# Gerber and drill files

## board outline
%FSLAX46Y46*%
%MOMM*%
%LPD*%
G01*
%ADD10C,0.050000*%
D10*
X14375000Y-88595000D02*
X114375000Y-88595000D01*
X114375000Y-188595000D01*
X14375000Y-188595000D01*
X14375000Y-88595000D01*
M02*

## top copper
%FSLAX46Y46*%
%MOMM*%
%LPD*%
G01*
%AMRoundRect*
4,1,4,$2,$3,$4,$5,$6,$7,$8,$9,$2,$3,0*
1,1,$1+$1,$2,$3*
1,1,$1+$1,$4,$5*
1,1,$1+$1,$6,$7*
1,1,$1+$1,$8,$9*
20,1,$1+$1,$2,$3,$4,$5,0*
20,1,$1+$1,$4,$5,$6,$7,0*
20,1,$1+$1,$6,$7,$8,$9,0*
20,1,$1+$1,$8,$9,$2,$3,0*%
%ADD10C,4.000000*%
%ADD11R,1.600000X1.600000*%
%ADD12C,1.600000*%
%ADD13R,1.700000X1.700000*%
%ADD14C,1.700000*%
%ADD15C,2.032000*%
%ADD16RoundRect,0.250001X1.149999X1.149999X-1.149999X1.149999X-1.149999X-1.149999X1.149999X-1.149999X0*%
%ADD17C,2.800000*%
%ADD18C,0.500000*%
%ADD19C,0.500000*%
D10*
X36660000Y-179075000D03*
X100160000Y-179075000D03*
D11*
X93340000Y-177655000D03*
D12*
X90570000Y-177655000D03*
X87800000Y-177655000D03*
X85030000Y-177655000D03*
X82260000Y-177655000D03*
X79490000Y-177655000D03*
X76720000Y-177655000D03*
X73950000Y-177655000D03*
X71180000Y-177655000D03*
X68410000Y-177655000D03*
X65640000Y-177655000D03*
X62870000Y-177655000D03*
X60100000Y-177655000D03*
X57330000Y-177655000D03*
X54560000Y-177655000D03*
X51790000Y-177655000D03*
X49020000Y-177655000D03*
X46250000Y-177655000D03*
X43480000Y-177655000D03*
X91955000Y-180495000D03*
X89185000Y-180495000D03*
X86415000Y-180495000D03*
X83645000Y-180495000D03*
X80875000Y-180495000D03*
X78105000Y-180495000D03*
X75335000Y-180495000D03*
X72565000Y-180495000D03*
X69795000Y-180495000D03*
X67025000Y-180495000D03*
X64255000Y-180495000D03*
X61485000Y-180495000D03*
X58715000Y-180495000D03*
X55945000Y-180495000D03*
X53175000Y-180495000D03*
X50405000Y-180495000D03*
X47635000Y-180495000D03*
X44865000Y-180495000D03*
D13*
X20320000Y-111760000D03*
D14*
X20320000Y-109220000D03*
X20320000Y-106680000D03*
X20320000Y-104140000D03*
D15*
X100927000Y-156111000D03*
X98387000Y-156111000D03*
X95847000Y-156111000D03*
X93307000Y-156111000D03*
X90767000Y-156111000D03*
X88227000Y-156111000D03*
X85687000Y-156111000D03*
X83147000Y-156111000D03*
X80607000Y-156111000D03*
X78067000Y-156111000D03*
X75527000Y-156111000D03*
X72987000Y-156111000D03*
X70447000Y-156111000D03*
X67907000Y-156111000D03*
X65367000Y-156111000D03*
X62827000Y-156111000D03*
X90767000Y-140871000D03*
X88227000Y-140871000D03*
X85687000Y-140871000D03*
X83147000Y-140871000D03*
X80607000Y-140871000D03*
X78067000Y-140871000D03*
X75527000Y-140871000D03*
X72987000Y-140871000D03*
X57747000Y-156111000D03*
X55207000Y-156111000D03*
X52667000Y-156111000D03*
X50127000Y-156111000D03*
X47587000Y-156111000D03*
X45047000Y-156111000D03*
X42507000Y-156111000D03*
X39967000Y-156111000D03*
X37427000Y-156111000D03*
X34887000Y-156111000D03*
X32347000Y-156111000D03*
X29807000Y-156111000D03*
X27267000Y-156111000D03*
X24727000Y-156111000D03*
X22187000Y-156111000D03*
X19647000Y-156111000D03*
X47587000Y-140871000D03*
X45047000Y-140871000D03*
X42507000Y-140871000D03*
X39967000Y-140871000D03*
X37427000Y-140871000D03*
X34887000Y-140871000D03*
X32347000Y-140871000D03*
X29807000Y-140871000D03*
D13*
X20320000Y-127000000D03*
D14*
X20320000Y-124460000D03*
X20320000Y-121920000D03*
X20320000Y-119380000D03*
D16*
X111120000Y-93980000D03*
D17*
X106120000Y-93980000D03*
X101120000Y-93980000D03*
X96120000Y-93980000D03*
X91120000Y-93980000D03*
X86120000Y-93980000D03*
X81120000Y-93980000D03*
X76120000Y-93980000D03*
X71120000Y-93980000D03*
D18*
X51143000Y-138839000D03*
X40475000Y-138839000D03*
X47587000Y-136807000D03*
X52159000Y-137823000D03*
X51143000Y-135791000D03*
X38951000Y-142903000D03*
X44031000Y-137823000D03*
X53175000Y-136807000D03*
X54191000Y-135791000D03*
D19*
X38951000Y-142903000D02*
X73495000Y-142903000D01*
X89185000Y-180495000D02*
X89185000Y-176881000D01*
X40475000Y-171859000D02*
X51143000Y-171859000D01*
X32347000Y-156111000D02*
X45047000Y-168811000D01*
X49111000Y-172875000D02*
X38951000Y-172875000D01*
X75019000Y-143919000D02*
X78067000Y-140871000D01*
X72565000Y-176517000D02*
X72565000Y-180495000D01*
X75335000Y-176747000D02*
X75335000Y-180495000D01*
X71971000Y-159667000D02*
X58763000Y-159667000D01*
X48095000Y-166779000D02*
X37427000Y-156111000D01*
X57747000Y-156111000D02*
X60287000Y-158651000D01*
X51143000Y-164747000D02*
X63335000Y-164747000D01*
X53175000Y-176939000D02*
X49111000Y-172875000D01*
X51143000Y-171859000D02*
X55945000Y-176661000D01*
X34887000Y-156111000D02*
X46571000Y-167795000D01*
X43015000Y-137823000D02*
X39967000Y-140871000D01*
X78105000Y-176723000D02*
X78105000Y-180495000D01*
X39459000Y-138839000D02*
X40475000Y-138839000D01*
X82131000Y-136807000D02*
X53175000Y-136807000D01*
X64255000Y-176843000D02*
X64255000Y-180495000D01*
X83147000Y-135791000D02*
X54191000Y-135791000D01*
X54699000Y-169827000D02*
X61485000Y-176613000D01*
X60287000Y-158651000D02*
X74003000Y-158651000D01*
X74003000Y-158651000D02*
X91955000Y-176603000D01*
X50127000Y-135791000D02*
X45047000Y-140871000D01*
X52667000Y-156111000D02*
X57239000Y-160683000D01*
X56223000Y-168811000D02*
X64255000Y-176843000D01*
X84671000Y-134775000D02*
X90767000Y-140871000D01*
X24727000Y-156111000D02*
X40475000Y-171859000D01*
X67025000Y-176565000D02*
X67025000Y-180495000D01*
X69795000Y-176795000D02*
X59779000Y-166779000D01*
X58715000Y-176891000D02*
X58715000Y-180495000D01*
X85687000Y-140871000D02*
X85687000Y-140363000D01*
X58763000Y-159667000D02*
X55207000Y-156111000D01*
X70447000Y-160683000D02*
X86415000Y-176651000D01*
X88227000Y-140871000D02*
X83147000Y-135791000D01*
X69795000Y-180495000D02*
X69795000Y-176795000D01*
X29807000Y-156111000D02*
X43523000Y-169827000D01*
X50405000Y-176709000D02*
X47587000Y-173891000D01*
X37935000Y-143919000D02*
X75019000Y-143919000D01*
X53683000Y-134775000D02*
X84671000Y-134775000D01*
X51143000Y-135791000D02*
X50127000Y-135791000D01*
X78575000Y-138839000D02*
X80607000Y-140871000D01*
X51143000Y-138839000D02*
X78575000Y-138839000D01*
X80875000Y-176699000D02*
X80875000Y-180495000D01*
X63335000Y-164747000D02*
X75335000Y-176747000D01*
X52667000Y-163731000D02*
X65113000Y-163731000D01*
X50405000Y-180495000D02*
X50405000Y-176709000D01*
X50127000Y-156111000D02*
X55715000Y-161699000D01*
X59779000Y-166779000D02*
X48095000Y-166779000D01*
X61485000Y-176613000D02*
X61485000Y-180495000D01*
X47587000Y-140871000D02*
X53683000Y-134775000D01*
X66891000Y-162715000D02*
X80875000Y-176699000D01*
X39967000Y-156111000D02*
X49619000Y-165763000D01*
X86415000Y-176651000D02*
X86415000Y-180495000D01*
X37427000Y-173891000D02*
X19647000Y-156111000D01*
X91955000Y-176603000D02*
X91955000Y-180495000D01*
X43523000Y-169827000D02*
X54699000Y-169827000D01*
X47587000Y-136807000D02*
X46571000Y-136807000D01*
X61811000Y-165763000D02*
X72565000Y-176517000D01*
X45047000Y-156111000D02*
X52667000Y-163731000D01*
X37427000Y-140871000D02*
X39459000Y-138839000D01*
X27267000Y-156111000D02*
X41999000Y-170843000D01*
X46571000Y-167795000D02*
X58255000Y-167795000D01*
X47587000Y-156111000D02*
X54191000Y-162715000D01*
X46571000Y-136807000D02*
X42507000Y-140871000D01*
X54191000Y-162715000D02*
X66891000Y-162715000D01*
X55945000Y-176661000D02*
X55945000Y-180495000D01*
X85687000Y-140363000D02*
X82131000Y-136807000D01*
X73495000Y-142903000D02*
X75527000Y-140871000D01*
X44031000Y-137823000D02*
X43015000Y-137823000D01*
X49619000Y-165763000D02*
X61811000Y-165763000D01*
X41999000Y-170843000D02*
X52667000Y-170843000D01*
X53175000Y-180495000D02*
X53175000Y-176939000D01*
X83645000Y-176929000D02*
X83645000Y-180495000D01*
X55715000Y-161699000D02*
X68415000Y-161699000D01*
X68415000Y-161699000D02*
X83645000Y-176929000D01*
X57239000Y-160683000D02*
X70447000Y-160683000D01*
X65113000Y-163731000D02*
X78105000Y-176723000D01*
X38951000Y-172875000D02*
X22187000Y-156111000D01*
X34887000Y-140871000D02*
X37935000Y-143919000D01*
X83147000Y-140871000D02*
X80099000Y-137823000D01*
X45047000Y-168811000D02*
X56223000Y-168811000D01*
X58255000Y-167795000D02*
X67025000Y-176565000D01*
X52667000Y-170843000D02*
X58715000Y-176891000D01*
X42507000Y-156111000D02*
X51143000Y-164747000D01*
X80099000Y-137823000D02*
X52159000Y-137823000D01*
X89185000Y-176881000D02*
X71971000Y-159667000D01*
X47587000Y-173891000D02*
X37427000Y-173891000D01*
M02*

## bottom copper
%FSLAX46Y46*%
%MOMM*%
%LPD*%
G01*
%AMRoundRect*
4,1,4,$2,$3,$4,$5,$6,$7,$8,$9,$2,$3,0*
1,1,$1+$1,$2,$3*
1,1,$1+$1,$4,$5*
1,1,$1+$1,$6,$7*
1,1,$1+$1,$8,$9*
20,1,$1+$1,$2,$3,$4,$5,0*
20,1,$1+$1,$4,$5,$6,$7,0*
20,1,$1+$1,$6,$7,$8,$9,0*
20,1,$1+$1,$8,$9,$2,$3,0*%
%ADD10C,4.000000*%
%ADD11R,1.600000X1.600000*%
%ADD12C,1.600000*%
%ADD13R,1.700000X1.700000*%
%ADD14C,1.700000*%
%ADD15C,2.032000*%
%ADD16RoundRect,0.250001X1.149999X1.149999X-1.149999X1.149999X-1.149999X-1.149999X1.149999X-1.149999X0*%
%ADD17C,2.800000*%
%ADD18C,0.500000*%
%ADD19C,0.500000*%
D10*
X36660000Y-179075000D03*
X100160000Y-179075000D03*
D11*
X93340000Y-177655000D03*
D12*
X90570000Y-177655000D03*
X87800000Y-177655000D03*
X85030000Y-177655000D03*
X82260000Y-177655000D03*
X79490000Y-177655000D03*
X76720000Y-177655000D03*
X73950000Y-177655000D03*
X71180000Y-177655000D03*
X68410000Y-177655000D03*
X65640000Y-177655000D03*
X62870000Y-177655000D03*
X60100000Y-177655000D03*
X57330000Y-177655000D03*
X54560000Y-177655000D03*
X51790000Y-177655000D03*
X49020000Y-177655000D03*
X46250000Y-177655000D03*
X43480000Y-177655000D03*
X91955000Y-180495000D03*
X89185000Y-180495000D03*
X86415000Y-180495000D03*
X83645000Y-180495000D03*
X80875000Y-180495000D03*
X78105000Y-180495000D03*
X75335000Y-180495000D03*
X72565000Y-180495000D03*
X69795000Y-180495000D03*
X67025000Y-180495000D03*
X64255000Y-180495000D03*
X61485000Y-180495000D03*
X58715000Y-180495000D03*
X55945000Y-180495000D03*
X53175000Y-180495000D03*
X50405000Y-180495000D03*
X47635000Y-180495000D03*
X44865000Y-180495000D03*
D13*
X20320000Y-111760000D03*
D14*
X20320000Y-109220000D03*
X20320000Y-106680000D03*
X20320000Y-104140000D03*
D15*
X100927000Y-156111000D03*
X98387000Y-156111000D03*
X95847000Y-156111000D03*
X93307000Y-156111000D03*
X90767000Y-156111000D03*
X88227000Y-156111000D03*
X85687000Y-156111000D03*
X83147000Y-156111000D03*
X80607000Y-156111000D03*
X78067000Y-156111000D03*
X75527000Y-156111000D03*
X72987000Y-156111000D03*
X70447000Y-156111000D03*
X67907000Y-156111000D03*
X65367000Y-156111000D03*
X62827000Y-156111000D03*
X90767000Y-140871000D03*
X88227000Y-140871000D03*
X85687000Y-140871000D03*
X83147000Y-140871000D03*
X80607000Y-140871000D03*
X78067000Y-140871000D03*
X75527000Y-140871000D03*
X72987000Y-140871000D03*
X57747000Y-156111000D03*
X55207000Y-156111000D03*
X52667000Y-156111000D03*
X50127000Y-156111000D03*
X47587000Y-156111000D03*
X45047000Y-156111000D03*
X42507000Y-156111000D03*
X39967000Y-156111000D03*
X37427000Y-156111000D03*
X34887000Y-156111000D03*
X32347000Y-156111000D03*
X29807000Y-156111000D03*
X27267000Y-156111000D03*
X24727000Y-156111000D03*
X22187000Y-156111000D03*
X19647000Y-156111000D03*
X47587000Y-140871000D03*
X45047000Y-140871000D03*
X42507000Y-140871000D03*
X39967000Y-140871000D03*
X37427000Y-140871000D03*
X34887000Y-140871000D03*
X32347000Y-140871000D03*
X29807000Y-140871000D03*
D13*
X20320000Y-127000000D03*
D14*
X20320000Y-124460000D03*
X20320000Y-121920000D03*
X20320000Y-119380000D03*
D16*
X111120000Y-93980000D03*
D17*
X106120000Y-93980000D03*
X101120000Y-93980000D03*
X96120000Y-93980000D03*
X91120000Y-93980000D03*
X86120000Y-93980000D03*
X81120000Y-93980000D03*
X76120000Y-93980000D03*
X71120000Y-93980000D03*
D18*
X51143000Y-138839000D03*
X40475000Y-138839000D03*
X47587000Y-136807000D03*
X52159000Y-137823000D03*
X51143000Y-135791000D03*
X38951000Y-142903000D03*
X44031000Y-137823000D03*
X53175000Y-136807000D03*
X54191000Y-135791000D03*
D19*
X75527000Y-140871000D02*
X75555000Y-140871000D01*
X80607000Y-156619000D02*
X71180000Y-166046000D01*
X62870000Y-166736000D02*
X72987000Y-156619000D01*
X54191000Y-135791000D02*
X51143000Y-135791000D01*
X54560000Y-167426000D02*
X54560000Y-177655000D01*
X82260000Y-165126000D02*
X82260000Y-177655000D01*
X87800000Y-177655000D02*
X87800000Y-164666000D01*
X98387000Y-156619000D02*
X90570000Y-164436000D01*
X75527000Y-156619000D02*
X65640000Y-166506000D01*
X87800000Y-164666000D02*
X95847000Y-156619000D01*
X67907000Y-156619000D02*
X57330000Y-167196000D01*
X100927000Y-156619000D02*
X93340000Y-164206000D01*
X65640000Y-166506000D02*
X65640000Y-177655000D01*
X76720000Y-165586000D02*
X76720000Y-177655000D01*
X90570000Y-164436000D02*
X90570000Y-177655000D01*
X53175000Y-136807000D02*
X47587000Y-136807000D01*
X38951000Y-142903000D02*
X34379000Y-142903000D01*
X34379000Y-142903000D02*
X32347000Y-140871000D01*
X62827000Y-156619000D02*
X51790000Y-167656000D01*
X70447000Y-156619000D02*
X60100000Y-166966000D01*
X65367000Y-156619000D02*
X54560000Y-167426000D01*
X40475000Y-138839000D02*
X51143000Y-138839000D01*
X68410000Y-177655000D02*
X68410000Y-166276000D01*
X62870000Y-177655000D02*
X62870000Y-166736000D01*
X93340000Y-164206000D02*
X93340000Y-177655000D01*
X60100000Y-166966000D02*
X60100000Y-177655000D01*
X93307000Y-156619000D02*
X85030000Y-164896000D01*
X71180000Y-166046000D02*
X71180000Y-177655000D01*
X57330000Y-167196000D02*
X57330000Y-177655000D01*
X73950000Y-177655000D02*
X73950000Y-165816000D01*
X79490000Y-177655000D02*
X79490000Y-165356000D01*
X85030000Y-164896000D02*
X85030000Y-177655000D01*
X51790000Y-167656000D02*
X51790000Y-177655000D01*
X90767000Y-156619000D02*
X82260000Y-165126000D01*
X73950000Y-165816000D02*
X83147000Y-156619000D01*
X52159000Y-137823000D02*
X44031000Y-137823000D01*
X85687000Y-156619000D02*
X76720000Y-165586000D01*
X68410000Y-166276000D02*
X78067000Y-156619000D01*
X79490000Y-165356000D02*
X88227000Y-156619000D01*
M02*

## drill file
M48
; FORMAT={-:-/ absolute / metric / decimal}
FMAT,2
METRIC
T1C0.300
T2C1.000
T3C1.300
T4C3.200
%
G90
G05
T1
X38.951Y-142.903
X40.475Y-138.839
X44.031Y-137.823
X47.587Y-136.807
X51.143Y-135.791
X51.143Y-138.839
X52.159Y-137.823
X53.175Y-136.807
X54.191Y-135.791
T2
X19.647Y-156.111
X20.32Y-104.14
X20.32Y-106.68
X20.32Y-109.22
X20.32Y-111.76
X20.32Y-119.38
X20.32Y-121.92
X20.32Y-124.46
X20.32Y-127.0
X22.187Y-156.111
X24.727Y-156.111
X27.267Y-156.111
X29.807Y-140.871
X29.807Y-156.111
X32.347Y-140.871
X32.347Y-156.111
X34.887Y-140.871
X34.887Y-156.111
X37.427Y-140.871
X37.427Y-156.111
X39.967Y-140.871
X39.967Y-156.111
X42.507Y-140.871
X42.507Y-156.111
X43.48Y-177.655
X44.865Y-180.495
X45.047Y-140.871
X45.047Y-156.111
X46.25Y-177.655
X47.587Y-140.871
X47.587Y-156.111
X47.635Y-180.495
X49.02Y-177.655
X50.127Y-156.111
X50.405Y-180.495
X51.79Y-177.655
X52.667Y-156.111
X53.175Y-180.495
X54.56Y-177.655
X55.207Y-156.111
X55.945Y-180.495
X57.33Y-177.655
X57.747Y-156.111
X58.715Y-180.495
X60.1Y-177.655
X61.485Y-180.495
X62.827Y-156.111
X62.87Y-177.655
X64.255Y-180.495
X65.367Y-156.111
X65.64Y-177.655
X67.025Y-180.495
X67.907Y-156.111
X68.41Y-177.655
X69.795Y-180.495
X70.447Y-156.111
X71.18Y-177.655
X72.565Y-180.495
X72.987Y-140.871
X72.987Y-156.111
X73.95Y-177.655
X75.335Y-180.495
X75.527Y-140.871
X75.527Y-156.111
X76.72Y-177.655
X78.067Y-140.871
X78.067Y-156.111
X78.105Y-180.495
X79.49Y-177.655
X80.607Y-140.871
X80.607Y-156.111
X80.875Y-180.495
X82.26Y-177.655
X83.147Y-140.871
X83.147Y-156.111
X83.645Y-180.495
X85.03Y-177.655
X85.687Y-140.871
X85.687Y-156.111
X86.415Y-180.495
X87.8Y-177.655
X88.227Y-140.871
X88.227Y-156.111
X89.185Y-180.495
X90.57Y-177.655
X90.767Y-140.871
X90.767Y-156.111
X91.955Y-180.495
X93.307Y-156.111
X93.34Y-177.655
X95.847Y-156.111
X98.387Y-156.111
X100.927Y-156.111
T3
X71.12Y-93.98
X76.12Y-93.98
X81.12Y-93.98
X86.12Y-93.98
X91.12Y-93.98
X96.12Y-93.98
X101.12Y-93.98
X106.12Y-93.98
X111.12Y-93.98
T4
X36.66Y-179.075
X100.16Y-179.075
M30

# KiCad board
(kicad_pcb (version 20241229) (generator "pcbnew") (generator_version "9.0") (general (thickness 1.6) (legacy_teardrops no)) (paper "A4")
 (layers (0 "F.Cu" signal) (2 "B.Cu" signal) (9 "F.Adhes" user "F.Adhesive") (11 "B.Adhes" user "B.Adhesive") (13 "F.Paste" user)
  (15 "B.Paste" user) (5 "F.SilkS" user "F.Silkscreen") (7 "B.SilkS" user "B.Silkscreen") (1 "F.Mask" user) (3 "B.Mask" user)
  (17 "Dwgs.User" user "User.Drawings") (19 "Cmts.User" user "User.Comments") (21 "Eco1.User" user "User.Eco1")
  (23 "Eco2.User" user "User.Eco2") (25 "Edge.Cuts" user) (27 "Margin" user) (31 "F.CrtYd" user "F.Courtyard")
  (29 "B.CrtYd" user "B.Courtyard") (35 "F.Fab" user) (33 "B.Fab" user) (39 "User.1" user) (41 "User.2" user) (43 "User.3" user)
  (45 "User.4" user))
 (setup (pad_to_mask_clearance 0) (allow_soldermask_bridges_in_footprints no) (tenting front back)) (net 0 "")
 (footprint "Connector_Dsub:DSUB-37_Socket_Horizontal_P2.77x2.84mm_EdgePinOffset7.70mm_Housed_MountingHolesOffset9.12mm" (layer "F.Cu")
  (at 93.34 177.655)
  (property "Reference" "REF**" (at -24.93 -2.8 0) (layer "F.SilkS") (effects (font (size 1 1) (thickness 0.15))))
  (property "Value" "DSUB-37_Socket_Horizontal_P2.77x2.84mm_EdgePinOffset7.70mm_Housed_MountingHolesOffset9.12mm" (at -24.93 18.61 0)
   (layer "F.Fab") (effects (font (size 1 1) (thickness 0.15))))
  (pad "0" thru_hole circle (at -56.68 1.42) (size 4 4) (drill 3.2) (layers "*.Cu" "*.Mask") (remove_unused_layers no))
  (pad "0" thru_hole circle (at 6.82 1.42) (size 4 4) (drill 3.2) (layers "*.Cu" "*.Mask") (remove_unused_layers no))
  (pad "1" thru_hole rect (at 0 0) (size 1.6 1.6) (drill 1) (layers "*.Cu" "*.Mask") (remove_unused_layers no))
  (pad "2" thru_hole circle (at -2.77 0) (size 1.6 1.6) (drill 1) (layers "*.Cu" "*.Mask") (remove_unused_layers no))
  (pad "3" thru_hole circle (at -5.54 0) (size 1.6 1.6) (drill 1) (layers "*.Cu" "*.Mask") (remove_unused_layers no))
  (pad "4" thru_hole circle (at -8.31 0) (size 1.6 1.6) (drill 1) (layers "*.Cu" "*.Mask") (remove_unused_layers no))
  (pad "5" thru_hole circle (at -11.08 0) (size 1.6 1.6) (drill 1) (layers "*.Cu" "*.Mask") (remove_unused_layers no))
  (pad "6" thru_hole circle (at -13.85 0) (size 1.6 1.6) (drill 1) (layers "*.Cu" "*.Mask") (remove_unused_layers no))
  (pad "7" thru_hole circle (at -16.62 0) (size 1.6 1.6) (drill 1) (layers "*.Cu" "*.Mask") (remove_unused_layers no))
  (pad "8" thru_hole circle (at -19.39 0) (size 1.6 1.6) (drill 1) (layers "*.Cu" "*.Mask") (remove_unused_layers no))
  (pad "9" thru_hole circle (at -22.16 0) (size 1.6 1.6) (drill 1) (layers "*.Cu" "*.Mask") (remove_unused_layers no))
  (pad "10" thru_hole circle (at -24.93 0) (size 1.6 1.6) (drill 1) (layers "*.Cu" "*.Mask") (remove_unused_layers no))
  (pad "11" thru_hole circle (at -27.7 0) (size 1.6 1.6) (drill 1) (layers "*.Cu" "*.Mask") (remove_unused_layers no))
  (pad "12" thru_hole circle (at -30.47 0) (size 1.6 1.6) (drill 1) (layers "*.Cu" "*.Mask") (remove_unused_layers no))
  (pad "13" thru_hole circle (at -33.24 0) (size 1.6 1.6) (drill 1) (layers "*.Cu" "*.Mask") (remove_unused_layers no))
  (pad "14" thru_hole circle (at -36.01 0) (size 1.6 1.6) (drill 1) (layers "*.Cu" "*.Mask") (remove_unused_layers no))
  (pad "15" thru_hole circle (at -38.78 0) (size 1.6 1.6) (drill 1) (layers "*.Cu" "*.Mask") (remove_unused_layers no))
  (pad "16" thru_hole circle (at -41.55 0) (size 1.6 1.6) (drill 1) (layers "*.Cu" "*.Mask") (remove_unused_layers no))
  (pad "17" thru_hole circle (at -44.32 0) (size 1.6 1.6) (drill 1) (layers "*.Cu" "*.Mask") (remove_unused_layers no))
  (pad "18" thru_hole circle (at -47.09 0) (size 1.6 1.6) (drill 1) (layers "*.Cu" "*.Mask") (remove_unused_layers no))
  (pad "19" thru_hole circle (at -49.86 0) (size 1.6 1.6) (drill 1) (layers "*.Cu" "*.Mask") (remove_unused_layers no))
  (pad "20" thru_hole circle (at -1.385 2.84) (size 1.6 1.6) (drill 1) (layers "*.Cu" "*.Mask") (remove_unused_layers no))
  (pad "21" thru_hole circle (at -4.155 2.84) (size 1.6 1.6) (drill 1) (layers "*.Cu" "*.Mask") (remove_unused_layers no))
  (pad "22" thru_hole circle (at -6.925 2.84) (size 1.6 1.6) (drill 1) (layers "*.Cu" "*.Mask") (remove_unused_layers no))
  (pad "23" thru_hole circle (at -9.695 2.84) (size 1.6 1.6) (drill 1) (layers "*.Cu" "*.Mask") (remove_unused_layers no))
  (pad "24" thru_hole circle (at -12.465 2.84) (size 1.6 1.6) (drill 1) (layers "*.Cu" "*.Mask") (remove_unused_layers no))
  (pad "25" thru_hole circle (at -15.235 2.84) (size 1.6 1.6) (drill 1) (layers "*.Cu" "*.Mask") (remove_unused_layers no))
  (pad "26" thru_hole circle (at -18.005 2.84) (size 1.6 1.6) (drill 1) (layers "*.Cu" "*.Mask") (remove_unused_layers no))
  (pad "27" thru_hole circle (at -20.775 2.84) (size 1.6 1.6) (drill 1) (layers "*.Cu" "*.Mask") (remove_unused_layers no))
  (pad "28" thru_hole circle (at -23.545 2.84) (size 1.6 1.6) (drill 1) (layers "*.Cu" "*.Mask") (remove_unused_layers no))
  (pad "29" thru_hole circle (at -26.315 2.84) (size 1.6 1.6) (drill 1) (layers "*.Cu" "*.Mask") (remove_unused_layers no))
  (pad "30" thru_hole circle (at -29.085 2.84) (size 1.6 1.6) (drill 1) (layers "*.Cu" "*.Mask") (remove_unused_layers no))
  (pad "31" thru_hole circle (at -31.855 2.84) (size 1.6 1.6) (drill 1) (layers "*.Cu" "*.Mask") (remove_unused_layers no))
  (pad "32" thru_hole circle (at -34.625 2.84) (size 1.6 1.6) (drill 1) (layers "*.Cu" "*.Mask") (remove_unused_layers no))
  (pad "33" thru_hole circle (at -37.395 2.84) (size 1.6 1.6) (drill 1) (layers "*.Cu" "*.Mask") (remove_unused_layers no))
  (pad "34" thru_hole circle (at -40.165 2.84) (size 1.6 1.6) (drill 1) (layers "*.Cu" "*.Mask") (remove_unused_layers no))
  (pad "35" thru_hole circle (at -42.935 2.84) (size 1.6 1.6) (drill 1) (layers "*.Cu" "*.Mask") (remove_unused_layers no))
  (pad "36" thru_hole circle (at -45.705 2.84) (size 1.6 1.6) (drill 1) (layers "*.Cu" "*.Mask") (remove_unused_layers no))
  (pad "37" thru_hole circle (at -48.475 2.84) (size 1.6 1.6) (drill 1) (layers "*.Cu" "*.Mask") (remove_unused_layers no)))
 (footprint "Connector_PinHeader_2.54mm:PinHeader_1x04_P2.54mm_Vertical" (layer "F.Cu") (at 20.32 111.76 180)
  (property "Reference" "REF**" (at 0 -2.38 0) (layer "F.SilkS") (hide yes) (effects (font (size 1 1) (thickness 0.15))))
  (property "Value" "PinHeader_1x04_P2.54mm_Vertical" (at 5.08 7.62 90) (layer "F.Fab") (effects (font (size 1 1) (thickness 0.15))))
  (pad "1" thru_hole rect (at 0 0 180) (size 1.7 1.7) (drill 1) (layers "*.Cu" "*.Mask") (remove_unused_layers no))
  (pad "2" thru_hole circle (at 0 2.54 180) (size 1.7 1.7) (drill 1) (layers "*.Cu" "*.Mask") (remove_unused_layers no))
  (pad "3" thru_hole circle (at 0 5.08 180) (size 1.7 1.7) (drill 1) (layers "*.Cu" "*.Mask") (remove_unused_layers no))
  (pad "4" thru_hole circle (at 0 7.62 180) (size 1.7 1.7) (drill 1) (layers "*.Cu" "*.Mask") (remove_unused_layers no)))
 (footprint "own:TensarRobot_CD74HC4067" (layer "F.Cu") (at 80.607 148.491 180)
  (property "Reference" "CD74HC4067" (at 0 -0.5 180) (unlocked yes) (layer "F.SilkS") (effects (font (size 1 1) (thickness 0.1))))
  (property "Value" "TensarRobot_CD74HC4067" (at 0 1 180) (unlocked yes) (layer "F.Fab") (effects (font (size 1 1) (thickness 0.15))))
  (pad "1" thru_hole circle (at -20.32 -7.62 90) (size 2.032 2.032) (drill 1) (layers "*.Cu" "*.Mask") (remove_unused_layers no))
  (pad "2" thru_hole circle (at -17.78 -7.62 90) (size 2.032 2.032) (drill 1) (layers "*.Cu" "*.Mask") (remove_unused_layers no))
  (pad "3" thru_hole circle (at -15.24 -7.62 90) (size 2.032 2.032) (drill 1) (layers "*.Cu" "*.Mask") (remove_unused_layers no))
  (pad "4" thru_hole circle (at -12.7 -7.62 90) (size 2.032 2.032) (drill 1) (layers "*.Cu" "*.Mask") (remove_unused_layers no))
  (pad "5" thru_hole circle (at -10.16 -7.62 90) (size 2.032 2.032) (drill 1) (layers "*.Cu" "*.Mask") (remove_unused_layers no))
  (pad "6" thru_hole circle (at -7.62 -7.62 90) (size 2.032 2.032) (drill 1) (layers "*.Cu" "*.Mask") (remove_unused_layers no))
  (pad "7" thru_hole circle (at -5.08 -7.62 90) (size 2.032 2.032) (drill 1) (layers "*.Cu" "*.Mask") (remove_unused_layers no))
  (pad "8" thru_hole circle (at -2.54 -7.62 90) (size 2.032 2.032) (drill 1) (layers "*.Cu" "*.Mask") (remove_unused_layers no))
  (pad "9" thru_hole circle (at 0 -7.62 90) (size 2.032 2.032) (drill 1) (layers "*.Cu" "*.Mask") (remove_unused_layers no))
  (pad "10" thru_hole circle (at 2.54 -7.62 90) (size 2.032 2.032) (drill 1) (layers "*.Cu" "*.Mask") (remove_unused_layers no))
  (pad "11" thru_hole circle (at 5.08 -7.62 90) (size 2.032 2.032) (drill 1) (layers "*.Cu" "*.Mask") (remove_unused_layers no))
  (pad "12" thru_hole circle (at 7.62 -7.62 90) (size 2.032 2.032) (drill 1) (layers "*.Cu" "*.Mask") (remove_unused_layers no))
  (pad "13" thru_hole circle (at 10.16 -7.62 90) (size 2.032 2.032) (drill 1) (layers "*.Cu" "*.Mask") (remove_unused_layers no))
  (pad "14" thru_hole circle (at 12.7 -7.62 90) (size 2.032 2.032) (drill 1) (layers "*.Cu" "*.Mask") (remove_unused_layers no))
  (pad "15" thru_hole circle (at 15.24 -7.62 90) (size 2.032 2.032) (drill 1) (layers "*.Cu" "*.Mask") (remove_unused_layers no))
  (pad "16" thru_hole circle (at 17.78 -7.62 90) (size 2.032 2.032) (drill 1) (layers "*.Cu" "*.Mask") (remove_unused_layers no))
  (pad "18" thru_hole circle (at -10.16 7.62 90) (size 2.032 2.032) (drill 1) (layers "*.Cu" "*.Mask") (remove_unused_layers no))
  (pad "19" thru_hole circle (at -7.62 7.62 90) (size 2.032 2.032) (drill 1) (layers "*.Cu" "*.Mask") (remove_unused_layers no))
  (pad "20" thru_hole circle (at -5.08 7.62 90) (size 2.032 2.032) (drill 1) (layers "*.Cu" "*.Mask") (remove_unused_layers no))
  (pad "21" thru_hole circle (at -2.54 7.62 90) (size 2.032 2.032) (drill 1) (layers "*.Cu" "*.Mask") (remove_unused_layers no))
  (pad "22" thru_hole circle (at 0 7.62 90) (size 2.032 2.032) (drill 1) (layers "*.Cu" "*.Mask") (remove_unused_layers no))
  (pad "23" thru_hole circle (at 2.54 7.62 90) (size 2.032 2.032) (drill 1) (layers "*.Cu" "*.Mask") (remove_unused_layers no))
  (pad "24" thru_hole circle (at 5.08 7.62 90) (size 2.032 2.032) (drill 1) (layers "*.Cu" "*.Mask") (remove_unused_layers no))
  (pad "25" thru_hole circle (at 7.62 7.62 90) (size 2.032 2.032) (drill 1) (layers "*.Cu" "*.Mask") (remove_unused_layers no)))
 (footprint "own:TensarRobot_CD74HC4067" (layer "F.Cu") (at 37.427 148.491 180)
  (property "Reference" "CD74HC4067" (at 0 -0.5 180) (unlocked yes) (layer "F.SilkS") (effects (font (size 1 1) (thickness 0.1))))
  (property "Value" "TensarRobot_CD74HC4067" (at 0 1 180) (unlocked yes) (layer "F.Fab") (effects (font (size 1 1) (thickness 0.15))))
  (pad "1" thru_hole circle (at -20.32 -7.62 90) (size 2.032 2.032) (drill 1) (layers "*.Cu" "*.Mask") (remove_unused_layers no))
  (pad "2" thru_hole circle (at -17.78 -7.62 90) (size 2.032 2.032) (drill 1) (layers "*.Cu" "*.Mask") (remove_unused_layers no))
  (pad "3" thru_hole circle (at -15.24 -7.62 90) (size 2.032 2.032) (drill 1) (layers "*.Cu" "*.Mask") (remove_unused_layers no))
  (pad "4" thru_hole circle (at -12.7 -7.62 90) (size 2.032 2.032) (drill 1) (layers "*.Cu" "*.Mask") (remove_unused_layers no))
  (pad "5" thru_hole circle (at -10.16 -7.62 90) (size 2.032 2.032) (drill 1) (layers "*.Cu" "*.Mask") (remove_unused_layers no))
  (pad "6" thru_hole circle (at -7.62 -7.62 90) (size 2.032 2.032) (drill 1) (layers "*.Cu" "*.Mask") (remove_unused_layers no))
  (pad "7" thru_hole circle (at -5.08 -7.62 90) (size 2.032 2.032) (drill 1) (layers "*.Cu" "*.Mask") (remove_unused_layers no))
  (pad "8" thru_hole circle (at -2.54 -7.62 90) (size 2.032 2.032) (drill 1) (layers "*.Cu" "*.Mask") (remove_unused_layers no))
  (pad "9" thru_hole circle (at 0 -7.62 90) (size 2.032 2.032) (drill 1) (layers "*.Cu" "*.Mask") (remove_unused_layers no))
  (pad "10" thru_hole circle (at 2.54 -7.62 90) (size 2.032 2.032) (drill 1) (layers "*.Cu" "*.Mask") (remove_unused_layers no))
  (pad "11" thru_hole circle (at 5.08 -7.62 90) (size 2.032 2.032) (drill 1) (layers "*.Cu" "*.Mask") (remove_unused_layers no))
  (pad "12" thru_hole circle (at 7.62 -7.62 90) (size 2.032 2.032) (drill 1) (layers "*.Cu" "*.Mask") (remove_unused_layers no))
  (pad "13" thru_hole circle (at 10.16 -7.62 90) (size 2.032 2.032) (drill 1) (layers "*.Cu" "*.Mask") (remove_unused_layers no))
  (pad "14" thru_hole circle (at 12.7 -7.62 90) (size 2.032 2.032) (drill 1) (layers "*.Cu" "*.Mask") (remove_unused_layers no))
  (pad "15" thru_hole circle (at 15.24 -7.62 90) (size 2.032 2.032) (drill 1) (layers "*.Cu" "*.Mask") (remove_unused_layers no))
  (pad "16" thru_hole circle (at 17.78 -7.62 90) (size 2.032 2.032) (drill 1) (layers "*.Cu" "*.Mask") (remove_unused_layers no))
  (pad "18" thru_hole circle (at -10.16 7.62 90) (size 2.032 2.032) (drill 1) (layers "*.Cu" "*.Mask") (remove_unused_layers no))
  (pad "19" thru_hole circle (at -7.62 7.62 90) (size 2.032 2.032) (drill 1) (layers "*.Cu" "*.Mask") (remove_unused_layers no))
  (pad "20" thru_hole circle (at -5.08 7.62 90) (size 2.032 2.032) (drill 1) (layers "*.Cu" "*.Mask") (remove_unused_layers no))
  (pad "21" thru_hole circle (at -2.54 7.62 90) (size 2.032 2.032) (drill 1) (layers "*.Cu" "*.Mask") (remove_unused_layers no))
  (pad "22" thru_hole circle (at 0 7.62 90) (size 2.032 2.032) (drill 1) (layers "*.Cu" "*.Mask") (remove_unused_layers no))
  (pad "23" thru_hole circle (at 2.54 7.62 90) (size 2.032 2.032) (drill 1) (layers "*.Cu" "*.Mask") (remove_unused_layers no))
  (pad "24" thru_hole circle (at 5.08 7.62 90) (size 2.032 2.032) (drill 1) (layers "*.Cu" "*.Mask") (remove_unused_layers no))
  (pad "25" thru_hole circle (at 7.62 7.62 90) (size 2.032 2.032) (drill 1) (layers "*.Cu" "*.Mask") (remove_unused_layers no)))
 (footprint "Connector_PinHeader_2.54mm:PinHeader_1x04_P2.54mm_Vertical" (layer "F.Cu") (at 20.32 127 180)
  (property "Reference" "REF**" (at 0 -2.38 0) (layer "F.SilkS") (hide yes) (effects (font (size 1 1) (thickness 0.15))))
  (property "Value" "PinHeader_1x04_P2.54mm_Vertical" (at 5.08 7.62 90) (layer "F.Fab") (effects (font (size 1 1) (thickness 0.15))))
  (pad "1" thru_hole rect (at 0 0 180) (size 1.7 1.7) (drill 1) (layers "*.Cu" "*.Mask") (remove_unused_layers no))
  (pad "2" thru_hole circle (at 0 2.54 180) (size 1.7 1.7) (drill 1) (layers "*.Cu" "*.Mask") (remove_unused_layers no))
  (pad "3" thru_hole circle (at 0 5.08 180) (size 1.7 1.7) (drill 1) (layers "*.Cu" "*.Mask") (remove_unused_layers no))
  (pad "4" thru_hole circle (at 0 7.62 180) (size 1.7 1.7) (drill 1) (layers "*.Cu" "*.Mask") (remove_unused_layers no)))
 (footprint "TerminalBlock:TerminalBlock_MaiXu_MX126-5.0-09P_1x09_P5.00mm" (layer "F.Cu") (at 111.12 93.98 180)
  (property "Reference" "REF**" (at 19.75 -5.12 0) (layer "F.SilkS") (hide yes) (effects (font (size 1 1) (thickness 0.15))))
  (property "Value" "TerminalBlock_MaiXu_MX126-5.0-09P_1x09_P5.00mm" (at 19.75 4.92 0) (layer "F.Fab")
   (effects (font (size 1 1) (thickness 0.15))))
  (pad "1" thru_hole roundrect (at 0 0 180) (size 2.8 2.8) (drill 1.3) (layers "*.Cu" "*.Mask") (remove_unused_layers no)
   (roundrect_rratio 0.089286))
  (pad "2" thru_hole circle (at 5 0 180) (size 2.8 2.8) (drill 1.3) (layers "*.Cu" "*.Mask") (remove_unused_layers no))
  (pad "3" thru_hole circle (at 10 0 180) (size 2.8 2.8) (drill 1.3) (layers "*.Cu" "*.Mask") (remove_unused_layers no))
  (pad "4" thru_hole circle (at 15 0 180) (size 2.8 2.8) (drill 1.3) (layers "*.Cu" "*.Mask") (remove_unused_layers no))
  (pad "5" thru_hole circle (at 20 0 180) (size 2.8 2.8) (drill 1.3) (layers "*.Cu" "*.Mask") (remove_unused_layers no))
  (pad "6" thru_hole circle (at 25 0 180) (size 2.8 2.8) (drill 1.3) (layers "*.Cu" "*.Mask") (remove_unused_layers no))
  (pad "7" thru_hole circle (at 30 0 180) (size 2.8 2.8) (drill 1.3) (layers "*.Cu" "*.Mask") (remove_unused_layers no))
  (pad "8" thru_hole circle (at 35 0 180) (size 2.8 2.8) (drill 1.3) (layers "*.Cu" "*.Mask") (remove_unused_layers no))
  (pad "9" thru_hole circle (at 40 0 180) (size 2.8 2.8) (drill 1.3) (layers "*.Cu" "*.Mask") (remove_unused_layers no)))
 (gr_rect (start 14.375 88.595) (end 114.375 188.595) (stroke (width 0.05) (type solid)) (fill no) (layer "Edge.Cuts"))
 (segment (start 38.951 142.903) (end 73.495 142.903) (width 0.5) (layer "F.Cu") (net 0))
 (segment (start 89.185 180.495) (end 89.185 176.881) (width 0.5) (layer "F.Cu") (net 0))
 (segment (start 40.475 171.859) (end 51.143 171.859) (width 0.5) (layer "F.Cu") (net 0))
 (segment (start 32.347 156.111) (end 45.047 168.811) (width 0.5) (layer "F.Cu") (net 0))
 (segment (start 49.111 172.875) (end 38.951 172.875) (width 0.5) (layer "F.Cu") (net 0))
 (segment (start 75.019 143.919) (end 78.067 140.871) (width 0.5) (layer "F.Cu") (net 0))
 (segment (start 72.565 176.517) (end 72.565 180.495) (width 0.5) (layer "F.Cu") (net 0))
 (segment (start 75.335 176.747) (end 75.335 180.495) (width 0.5) (layer "F.Cu") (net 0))
 (segment (start 71.971 159.667) (end 58.763 159.667) (width 0.5) (layer "F.Cu") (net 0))
 (segment (start 48.095 166.779) (end 37.427 156.111) (width 0.5) (layer "F.Cu") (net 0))
 (segment (start 57.747 156.111) (end 60.287 158.651) (width 0.5) (layer "F.Cu") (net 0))
 (segment (start 51.143 164.747) (end 63.335 164.747) (width 0.5) (layer "F.Cu") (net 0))
 (segment (start 53.175 176.939) (end 49.111 172.875) (width 0.5) (layer "F.Cu") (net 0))
 (segment (start 51.143 171.859) (end 55.945 176.661) (width 0.5) (layer "F.Cu") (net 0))
 (segment (start 34.887 156.111) (end 46.571 167.795) (width 0.5) (layer "F.Cu") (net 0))
 (segment (start 43.015 137.823) (end 39.967 140.871) (width 0.5) (layer "F.Cu") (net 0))
 (segment (start 78.105 176.723) (end 78.105 180.495) (width 0.5) (layer "F.Cu") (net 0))
 (segment (start 39.459 138.839) (end 40.475 138.839) (width 0.5) (layer "F.Cu") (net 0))
 (segment (start 82.131 136.807) (end 53.175 136.807) (width 0.5) (layer "F.Cu") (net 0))
 (segment (start 64.255 176.843) (end 64.255 180.495) (width 0.5) (layer "F.Cu") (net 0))
 (segment (start 83.147 135.791) (end 54.191 135.791) (width 0.5) (layer "F.Cu") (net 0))
 (segment (start 54.699 169.827) (end 61.485 176.613) (width 0.5) (layer "F.Cu") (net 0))
 (segment (start 60.287 158.651) (end 74.003 158.651) (width 0.5) (layer "F.Cu") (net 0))
 (segment (start 74.003 158.651) (end 91.955 176.603) (width 0.5) (layer "F.Cu") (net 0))
 (segment (start 50.127 135.791) (end 45.047 140.871) (width 0.5) (layer "F.Cu") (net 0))
 (segment (start 52.667 156.111) (end 57.239 160.683) (width 0.5) (layer "F.Cu") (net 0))
 (segment (start 56.223 168.811) (end 64.255 176.843) (width 0.5) (layer "F.Cu") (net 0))
 (segment (start 84.671 134.775) (end 90.767 140.871) (width 0.5) (layer "F.Cu") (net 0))
 (segment (start 24.727 156.111) (end 40.475 171.859) (width 0.5) (layer "F.Cu") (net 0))
 (segment (start 67.025 176.565) (end 67.025 180.495) (width 0.5) (layer "F.Cu") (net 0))
 (segment (start 69.795 176.795) (end 59.779 166.779) (width 0.5) (layer "F.Cu") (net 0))
 (segment (start 58.715 176.891) (end 58.715 180.495) (width 0.5) (layer "F.Cu") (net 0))
 (segment (start 85.687 140.871) (end 85.687 140.363) (width 0.5) (layer "F.Cu") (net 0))
 (segment (start 58.763 159.667) (end 55.207 156.111) (width 0.5) (layer "F.Cu") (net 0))
 (segment (start 70.447 160.683) (end 86.415 176.651) (width 0.5) (layer "F.Cu") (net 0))
 (segment (start 88.227 140.871) (end 83.147 135.791) (width 0.5) (layer "F.Cu") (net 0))
 (segment (start 69.795 180.495) (end 69.795 176.795) (width 0.5) (layer "F.Cu") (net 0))
 (segment (start 29.807 156.111) (end 43.523 169.827) (width 0.5) (layer "F.Cu") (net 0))
 (segment (start 50.405 176.709) (end 47.587 173.891) (width 0.5) (layer "F.Cu") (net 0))
 (segment (start 37.935 143.919) (end 75.019 143.919) (width 0.5) (layer "F.Cu") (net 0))
 (segment (start 53.683 134.775) (end 84.671 134.775) (width 0.5) (layer "F.Cu") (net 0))
 (segment (start 51.143 135.791) (end 50.127 135.791) (width 0.5) (layer "F.Cu") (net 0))
 (segment (start 78.575 138.839) (end 80.607 140.871) (width 0.5) (layer "F.Cu") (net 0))
 (segment (start 51.143 138.839) (end 78.575 138.839) (width 0.5) (layer "F.Cu") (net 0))
 (segment (start 80.875 176.699) (end 80.875 180.495) (width 0.5) (layer "F.Cu") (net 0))
 (segment (start 63.335 164.747) (end 75.335 176.747) (width 0.5) (layer "F.Cu") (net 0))
 (segment (start 52.667 163.731) (end 65.113 163.731) (width 0.5) (layer "F.Cu") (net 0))
 (segment (start 50.405 180.495) (end 50.405 176.709) (width 0.5) (layer "F.Cu") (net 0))
 (segment (start 50.127 156.111) (end 55.715 161.699) (width 0.5) (layer "F.Cu") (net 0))
 (segment (start 59.779 166.779) (end 48.095 166.779) (width 0.5) (layer "F.Cu") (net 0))
 (segment (start 61.485 176.613) (end 61.485 180.495) (width 0.5) (layer "F.Cu") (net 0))
 (segment (start 47.587 140.871) (end 53.683 134.775) (width 0.5) (layer "F.Cu") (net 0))
 (segment (start 66.891 162.715) (end 80.875 176.699) (width 0.5) (layer "F.Cu") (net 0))
 (segment (start 39.967 156.111) (end 49.619 165.763) (width 0.5) (layer "F.Cu") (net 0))
 (segment (start 86.415 176.651) (end 86.415 180.495) (width 0.5) (layer "F.Cu") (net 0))
 (segment (start 37.427 173.891) (end 19.647 156.111) (width 0.5) (layer "F.Cu") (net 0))
 (segment (start 91.955 176.603) (end 91.955 180.495) (width 0.5) (layer "F.Cu") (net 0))
 (segment (start 43.523 169.827) (end 54.699 169.827) (width 0.5) (layer "F.Cu") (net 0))
 (segment (start 47.587 136.807) (end 46.571 136.807) (width 0.5) (layer "F.Cu") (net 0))
 (segment (start 61.811 165.763) (end 72.565 176.517) (width 0.5) (layer "F.Cu") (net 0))
 (segment (start 45.047 156.111) (end 52.667 163.731) (width 0.5) (layer "F.Cu") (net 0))
 (segment (start 37.427 140.871) (end 39.459 138.839) (width 0.5) (layer "F.Cu") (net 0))
 (segment (start 27.267 156.111) (end 41.999 170.843) (width 0.5) (layer "F.Cu") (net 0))
 (segment (start 46.571 167.795) (end 58.255 167.795) (width 0.5) (layer "F.Cu") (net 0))
 (segment (start 47.587 156.111) (end 54.191 162.715) (width 0.5) (layer "F.Cu") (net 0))
 (segment (start 46.571 136.807) (end 42.507 140.871) (width 0.5) (layer "F.Cu") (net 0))
 (segment (start 54.191 162.715) (end 66.891 162.715) (width 0.5) (layer "F.Cu") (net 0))
 (segment (start 55.945 176.661) (end 55.945 180.495) (width 0.5) (layer "F.Cu") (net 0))
 (segment (start 85.687 140.363) (end 82.131 136.807) (width 0.5) (layer "F.Cu") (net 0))
 (segment (start 73.495 142.903) (end 75.527 140.871) (width 0.5) (layer "F.Cu") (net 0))
 (segment (start 44.031 137.823) (end 43.015 137.823) (width 0.5) (layer "F.Cu") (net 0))
 (segment (start 49.619 165.763) (end 61.811 165.763) (width 0.5) (layer "F.Cu") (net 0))
 (segment (start 41.999 170.843) (end 52.667 170.843) (width 0.5) (layer "F.Cu") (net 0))
 (segment (start 53.175 180.495) (end 53.175 176.939) (width 0.5) (layer "F.Cu") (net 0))
 (segment (start 83.645 176.929) (end 83.645 180.495) (width 0.5) (layer "F.Cu") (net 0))
 (segment (start 55.715 161.699) (end 68.415 161.699) (width 0.5) (layer "F.Cu") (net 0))
 (segment (start 68.415 161.699) (end 83.645 176.929) (width 0.5) (layer "F.Cu") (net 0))
 (segment (start 57.239 160.683) (end 70.447 160.683) (width 0.5) (layer "F.Cu") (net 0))
 (segment (start 65.113 163.731) (end 78.105 176.723) (width 0.5) (layer "F.Cu") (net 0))
 (segment (start 38.951 172.875) (end 22.187 156.111) (width 0.5) (layer "F.Cu") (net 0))
 (segment (start 34.887 140.871) (end 37.935 143.919) (width 0.5) (layer "F.Cu") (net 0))
 (segment (start 83.147 140.871) (end 80.099 137.823) (width 0.5) (layer "F.Cu") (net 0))
 (segment (start 45.047 168.811) (end 56.223 168.811) (width 0.5) (layer "F.Cu") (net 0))
 (segment (start 58.255 167.795) (end 67.025 176.565) (width 0.5) (layer "F.Cu") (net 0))
 (segment (start 52.667 170.843) (end 58.715 176.891) (width 0.5) (layer "F.Cu") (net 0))
 (segment (start 42.507 156.111) (end 51.143 164.747) (width 0.5) (layer "F.Cu") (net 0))
 (segment (start 80.099 137.823) (end 52.159 137.823) (width 0.5) (layer "F.Cu") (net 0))
 (segment (start 89.185 176.881) (end 71.971 159.667) (width 0.5) (layer "F.Cu") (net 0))
 (segment (start 47.587 173.891) (end 37.427 173.891) (width 0.5) (layer "F.Cu") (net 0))
 (via (at 51.143 138.839) (size 0.5) (drill 0.3) (layers "F.Cu" "B.Cu") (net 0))
 (via (at 40.475 138.839) (size 0.5) (drill 0.3) (layers "F.Cu" "B.Cu") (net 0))
 (via (at 47.587 136.807) (size 0.5) (drill 0.3) (layers "F.Cu" "B.Cu") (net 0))
 (via (at 52.159 137.823) (size 0.5) (drill 0.3) (layers "F.Cu" "B.Cu") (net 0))
 (via (at 51.143 135.791) (size 0.5) (drill 0.3) (layers "F.Cu" "B.Cu") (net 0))
 (via (at 38.951 142.903) (size 0.5) (drill 0.3) (layers "F.Cu" "B.Cu") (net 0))
 (via (at 44.031 137.823) (size 0.5) (drill 0.3) (layers "F.Cu" "B.Cu") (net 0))
 (via (at 53.175 136.807) (size 0.5) (drill 0.3) (layers "F.Cu" "B.Cu") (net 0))
 (via (at 54.191 135.791) (size 0.5) (drill 0.3) (layers "F.Cu" "B.Cu") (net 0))
 (segment (start 75.527 140.871) (end 75.555 140.871) (width 0.5) (layer "B.Cu") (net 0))
 (segment (start 80.607 156.619) (end 71.18 166.046) (width 0.5) (layer "B.Cu") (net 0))
 (segment (start 62.87 166.736) (end 72.987 156.619) (width 0.5) (layer "B.Cu") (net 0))
 (segment (start 54.191 135.791) (end 51.143 135.791) (width 0.5) (layer "B.Cu") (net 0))
 (segment (start 54.56 167.426) (end 54.56 177.655) (width 0.5) (layer "B.Cu") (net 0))
 (segment (start 82.26 165.126) (end 82.26 177.655) (width 0.5) (layer "B.Cu") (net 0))
 (segment (start 87.8 177.655) (end 87.8 164.666) (width 0.5) (layer "B.Cu") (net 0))
 (segment (start 98.387 156.619) (end 90.57 164.436) (width 0.5) (layer "B.Cu") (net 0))
 (segment (start 75.527 156.619) (end 65.64 166.506) (width 0.5) (layer "B.Cu") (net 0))
 (segment (start 87.8 164.666) (end 95.847 156.619) (width 0.5) (layer "B.Cu") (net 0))
 (segment (start 67.907 156.619) (end 57.33 167.196) (width 0.5) (layer "B.Cu") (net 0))
 (segment (start 100.927 156.619) (end 93.34 164.206) (width 0.5) (layer "B.Cu") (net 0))
 (segment (start 65.64 166.506) (end 65.64 177.655) (width 0.5) (layer "B.Cu") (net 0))
 (segment (start 76.72 165.586) (end 76.72 177.655) (width 0.5) (layer "B.Cu") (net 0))
 (segment (start 90.57 164.436) (end 90.57 177.655) (width 0.5) (layer "B.Cu") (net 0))
 (segment (start 53.175 136.807) (end 47.587 136.807) (width 0.5) (layer "B.Cu") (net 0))
 (segment (start 38.951 142.903) (end 34.379 142.903) (width 0.5) (layer "B.Cu") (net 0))
 (segment (start 34.379 142.903) (end 32.347 140.871) (width 0.5) (layer "B.Cu") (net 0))
 (segment (start 62.827 156.619) (end 51.79 167.656) (width 0.5) (layer "B.Cu") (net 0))
 (segment (start 70.447 156.619) (end 60.1 166.966) (width 0.5) (layer "B.Cu") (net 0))
 (segment (start 65.367 156.619) (end 54.56 167.426) (width 0.5) (layer "B.Cu") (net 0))
 (segment (start 40.475 138.839) (end 51.143 138.839) (width 0.5) (layer "B.Cu") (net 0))
 (segment (start 68.41 177.655) (end 68.41 166.276) (width 0.5) (layer "B.Cu") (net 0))
 (segment (start 62.87 177.655) (end 62.87 166.736) (width 0.5) (layer "B.Cu") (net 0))
 (segment (start 93.34 164.206) (end 93.34 177.655) (width 0.5) (layer "B.Cu") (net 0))
 (segment (start 60.1 166.966) (end 60.1 177.655) (width 0.5) (layer "B.Cu") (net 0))
 (segment (start 93.307 156.619) (end 85.03 164.896) (width 0.5) (layer "B.Cu") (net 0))
 (segment (start 71.18 166.046) (end 71.18 177.655) (width 0.5) (layer "B.Cu") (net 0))
 (segment (start 57.33 167.196) (end 57.33 177.655) (width 0.5) (layer "B.Cu") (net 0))
 (segment (start 73.95 177.655) (end 73.95 165.816) (width 0.5) (layer "B.Cu") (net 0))
 (segment (start 79.49 177.655) (end 79.49 165.356) (width 0.5) (layer "B.Cu") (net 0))
 (segment (start 85.03 164.896) (end 85.03 177.655) (width 0.5) (layer "B.Cu") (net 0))
 (segment (start 51.79 167.656) (end 51.79 177.655) (width 0.5) (layer "B.Cu") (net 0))
 (segment (start 90.767 156.619) (end 82.26 165.126) (width 0.5) (layer "B.Cu") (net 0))
 (segment (start 73.95 165.816) (end 83.147 156.619) (width 0.5) (layer "B.Cu") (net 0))
 (segment (start 52.159 137.823) (end 44.031 137.823) (width 0.5) (layer "B.Cu") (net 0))
 (segment (start 85.687 156.619) (end 76.72 165.586) (width 0.5) (layer "B.Cu") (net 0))
 (segment (start 68.41 166.276) (end 78.067 156.619) (width 0.5) (layer "B.Cu") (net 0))
 (segment (start 79.49 165.356) (end 88.227 156.619) (width 0.5) (layer "B.Cu") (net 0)))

